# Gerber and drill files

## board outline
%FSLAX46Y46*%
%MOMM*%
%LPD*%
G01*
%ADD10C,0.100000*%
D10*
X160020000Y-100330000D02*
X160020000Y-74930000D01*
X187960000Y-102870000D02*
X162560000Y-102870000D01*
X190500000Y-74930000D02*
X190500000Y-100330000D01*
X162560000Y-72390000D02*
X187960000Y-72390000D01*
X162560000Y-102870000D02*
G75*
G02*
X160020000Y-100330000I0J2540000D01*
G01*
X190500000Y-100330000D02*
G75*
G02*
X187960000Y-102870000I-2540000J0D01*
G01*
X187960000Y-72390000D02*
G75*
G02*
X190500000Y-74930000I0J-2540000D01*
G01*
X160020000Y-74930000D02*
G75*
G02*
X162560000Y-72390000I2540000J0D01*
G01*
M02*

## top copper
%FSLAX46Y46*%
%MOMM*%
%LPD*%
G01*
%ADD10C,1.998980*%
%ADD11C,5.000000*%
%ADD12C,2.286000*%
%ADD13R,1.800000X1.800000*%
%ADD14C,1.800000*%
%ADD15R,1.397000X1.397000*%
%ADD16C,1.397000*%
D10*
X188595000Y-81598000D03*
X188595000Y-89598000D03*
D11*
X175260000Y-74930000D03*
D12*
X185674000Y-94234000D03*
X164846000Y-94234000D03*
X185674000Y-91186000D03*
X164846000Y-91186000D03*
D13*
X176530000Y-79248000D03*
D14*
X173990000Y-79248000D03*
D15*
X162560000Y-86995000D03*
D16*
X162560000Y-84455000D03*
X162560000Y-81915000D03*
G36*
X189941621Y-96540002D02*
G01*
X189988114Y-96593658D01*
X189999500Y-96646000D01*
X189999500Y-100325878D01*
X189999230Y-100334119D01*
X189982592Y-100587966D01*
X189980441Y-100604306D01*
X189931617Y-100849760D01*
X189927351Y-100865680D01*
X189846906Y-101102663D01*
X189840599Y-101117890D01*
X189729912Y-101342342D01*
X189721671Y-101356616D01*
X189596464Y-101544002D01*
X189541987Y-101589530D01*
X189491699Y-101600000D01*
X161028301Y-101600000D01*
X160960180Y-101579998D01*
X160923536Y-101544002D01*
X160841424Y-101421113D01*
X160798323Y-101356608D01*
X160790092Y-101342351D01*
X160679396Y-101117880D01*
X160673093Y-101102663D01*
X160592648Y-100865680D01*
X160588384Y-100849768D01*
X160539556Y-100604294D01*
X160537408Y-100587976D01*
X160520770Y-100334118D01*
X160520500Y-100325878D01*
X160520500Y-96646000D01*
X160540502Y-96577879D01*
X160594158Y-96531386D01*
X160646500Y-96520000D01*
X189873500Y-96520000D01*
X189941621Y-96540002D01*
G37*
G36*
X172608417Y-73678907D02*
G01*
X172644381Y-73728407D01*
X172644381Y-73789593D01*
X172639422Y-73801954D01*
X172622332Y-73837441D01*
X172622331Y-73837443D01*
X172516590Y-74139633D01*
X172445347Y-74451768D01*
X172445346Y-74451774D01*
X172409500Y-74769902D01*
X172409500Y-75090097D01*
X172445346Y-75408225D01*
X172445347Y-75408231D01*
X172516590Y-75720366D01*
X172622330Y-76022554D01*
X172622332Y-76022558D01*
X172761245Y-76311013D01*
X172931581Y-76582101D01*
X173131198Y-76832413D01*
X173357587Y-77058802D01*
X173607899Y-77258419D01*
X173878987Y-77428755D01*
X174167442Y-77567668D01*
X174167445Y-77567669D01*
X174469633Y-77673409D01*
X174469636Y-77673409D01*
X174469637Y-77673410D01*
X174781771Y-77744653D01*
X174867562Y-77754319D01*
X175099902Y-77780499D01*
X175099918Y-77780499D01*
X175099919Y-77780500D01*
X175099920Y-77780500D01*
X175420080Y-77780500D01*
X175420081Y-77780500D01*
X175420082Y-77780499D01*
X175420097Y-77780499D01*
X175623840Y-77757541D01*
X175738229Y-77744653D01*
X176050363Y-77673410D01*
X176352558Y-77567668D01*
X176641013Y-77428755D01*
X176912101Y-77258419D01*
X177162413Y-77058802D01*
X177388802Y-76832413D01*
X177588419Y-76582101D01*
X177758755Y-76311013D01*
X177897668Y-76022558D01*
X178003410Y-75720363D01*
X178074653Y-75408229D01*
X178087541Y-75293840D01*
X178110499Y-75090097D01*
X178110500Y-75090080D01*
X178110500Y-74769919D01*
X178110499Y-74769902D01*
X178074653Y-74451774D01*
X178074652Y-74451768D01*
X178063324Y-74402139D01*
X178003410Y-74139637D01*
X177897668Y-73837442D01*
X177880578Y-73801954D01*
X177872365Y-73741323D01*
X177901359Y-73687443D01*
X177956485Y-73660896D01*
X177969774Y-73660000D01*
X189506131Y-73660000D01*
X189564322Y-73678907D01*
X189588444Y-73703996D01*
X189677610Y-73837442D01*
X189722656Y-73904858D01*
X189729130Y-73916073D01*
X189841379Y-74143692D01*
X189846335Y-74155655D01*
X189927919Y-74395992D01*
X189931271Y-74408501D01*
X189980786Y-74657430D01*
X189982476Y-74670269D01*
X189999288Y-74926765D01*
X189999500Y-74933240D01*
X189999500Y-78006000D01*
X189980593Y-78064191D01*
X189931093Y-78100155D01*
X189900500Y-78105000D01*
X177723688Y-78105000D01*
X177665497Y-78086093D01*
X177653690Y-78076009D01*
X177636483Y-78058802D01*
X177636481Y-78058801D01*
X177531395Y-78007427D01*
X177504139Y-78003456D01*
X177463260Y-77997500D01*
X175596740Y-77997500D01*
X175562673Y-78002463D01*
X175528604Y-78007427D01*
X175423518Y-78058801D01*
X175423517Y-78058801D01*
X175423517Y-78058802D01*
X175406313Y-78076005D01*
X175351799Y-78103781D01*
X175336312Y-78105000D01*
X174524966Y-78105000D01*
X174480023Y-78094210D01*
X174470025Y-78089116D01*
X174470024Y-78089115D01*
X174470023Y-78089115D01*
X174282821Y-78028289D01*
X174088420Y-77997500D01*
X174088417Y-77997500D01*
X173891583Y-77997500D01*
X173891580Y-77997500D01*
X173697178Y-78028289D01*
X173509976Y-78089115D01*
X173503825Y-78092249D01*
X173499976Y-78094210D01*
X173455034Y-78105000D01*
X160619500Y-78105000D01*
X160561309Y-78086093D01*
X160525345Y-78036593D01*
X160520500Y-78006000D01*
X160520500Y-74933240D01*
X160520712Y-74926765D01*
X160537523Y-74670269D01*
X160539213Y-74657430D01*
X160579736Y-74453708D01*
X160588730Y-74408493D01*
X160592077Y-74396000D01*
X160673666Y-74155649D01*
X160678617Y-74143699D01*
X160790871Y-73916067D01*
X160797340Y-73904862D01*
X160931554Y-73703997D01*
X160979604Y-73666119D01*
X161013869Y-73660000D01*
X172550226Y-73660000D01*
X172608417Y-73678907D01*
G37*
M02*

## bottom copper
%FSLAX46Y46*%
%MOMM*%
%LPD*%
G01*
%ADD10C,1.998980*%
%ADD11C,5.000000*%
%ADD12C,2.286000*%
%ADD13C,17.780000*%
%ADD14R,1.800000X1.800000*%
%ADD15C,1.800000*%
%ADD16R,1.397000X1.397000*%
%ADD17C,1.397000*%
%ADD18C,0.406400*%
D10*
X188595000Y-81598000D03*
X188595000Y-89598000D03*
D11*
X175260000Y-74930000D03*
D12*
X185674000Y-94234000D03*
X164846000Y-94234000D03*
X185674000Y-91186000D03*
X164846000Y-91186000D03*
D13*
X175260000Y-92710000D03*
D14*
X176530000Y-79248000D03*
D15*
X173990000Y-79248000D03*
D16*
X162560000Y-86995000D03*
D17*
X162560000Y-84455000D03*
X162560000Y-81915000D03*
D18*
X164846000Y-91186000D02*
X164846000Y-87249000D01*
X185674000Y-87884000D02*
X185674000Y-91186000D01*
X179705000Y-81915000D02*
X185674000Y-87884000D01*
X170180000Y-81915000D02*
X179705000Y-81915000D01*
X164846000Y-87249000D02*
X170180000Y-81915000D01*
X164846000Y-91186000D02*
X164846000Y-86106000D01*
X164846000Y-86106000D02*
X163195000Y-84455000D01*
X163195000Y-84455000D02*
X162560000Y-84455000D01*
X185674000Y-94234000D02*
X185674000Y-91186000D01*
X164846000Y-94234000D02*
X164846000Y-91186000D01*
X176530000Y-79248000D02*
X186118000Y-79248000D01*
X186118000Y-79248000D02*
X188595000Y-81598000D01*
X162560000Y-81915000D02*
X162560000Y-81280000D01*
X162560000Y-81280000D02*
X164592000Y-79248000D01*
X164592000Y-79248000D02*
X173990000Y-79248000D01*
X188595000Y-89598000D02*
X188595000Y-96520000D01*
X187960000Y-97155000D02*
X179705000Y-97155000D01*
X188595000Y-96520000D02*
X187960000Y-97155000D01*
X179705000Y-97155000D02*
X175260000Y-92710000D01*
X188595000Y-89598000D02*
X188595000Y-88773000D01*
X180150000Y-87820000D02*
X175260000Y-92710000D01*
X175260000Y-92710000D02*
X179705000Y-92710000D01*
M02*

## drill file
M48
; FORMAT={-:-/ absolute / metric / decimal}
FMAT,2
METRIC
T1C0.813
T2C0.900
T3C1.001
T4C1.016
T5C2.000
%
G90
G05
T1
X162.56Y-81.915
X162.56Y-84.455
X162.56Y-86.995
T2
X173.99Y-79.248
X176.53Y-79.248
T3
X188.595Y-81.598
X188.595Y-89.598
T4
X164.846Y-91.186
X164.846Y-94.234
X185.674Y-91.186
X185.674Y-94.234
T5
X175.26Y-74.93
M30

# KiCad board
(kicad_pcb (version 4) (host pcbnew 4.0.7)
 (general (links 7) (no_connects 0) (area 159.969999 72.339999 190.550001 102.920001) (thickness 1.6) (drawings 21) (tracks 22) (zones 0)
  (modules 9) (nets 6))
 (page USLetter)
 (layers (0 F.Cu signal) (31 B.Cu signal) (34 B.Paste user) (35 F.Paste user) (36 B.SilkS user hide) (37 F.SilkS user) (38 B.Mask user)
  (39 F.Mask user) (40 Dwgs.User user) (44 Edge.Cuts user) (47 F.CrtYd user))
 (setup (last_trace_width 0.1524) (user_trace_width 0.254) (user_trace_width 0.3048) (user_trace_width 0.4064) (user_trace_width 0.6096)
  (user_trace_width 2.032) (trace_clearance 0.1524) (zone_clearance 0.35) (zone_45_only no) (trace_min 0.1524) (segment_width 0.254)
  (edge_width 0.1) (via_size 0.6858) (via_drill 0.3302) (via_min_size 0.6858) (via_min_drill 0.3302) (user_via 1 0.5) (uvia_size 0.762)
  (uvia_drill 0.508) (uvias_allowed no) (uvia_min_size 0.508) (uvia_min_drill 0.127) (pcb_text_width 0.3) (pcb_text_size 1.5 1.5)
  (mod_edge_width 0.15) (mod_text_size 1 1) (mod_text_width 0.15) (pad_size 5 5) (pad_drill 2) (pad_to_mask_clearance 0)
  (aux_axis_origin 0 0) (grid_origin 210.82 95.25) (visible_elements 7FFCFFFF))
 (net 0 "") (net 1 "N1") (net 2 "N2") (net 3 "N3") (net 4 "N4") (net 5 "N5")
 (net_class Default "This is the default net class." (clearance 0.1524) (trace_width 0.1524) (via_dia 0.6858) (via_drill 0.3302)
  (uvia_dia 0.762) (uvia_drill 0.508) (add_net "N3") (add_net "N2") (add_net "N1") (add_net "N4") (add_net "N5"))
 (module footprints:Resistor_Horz (layer F.Cu) (at 188.595 85.598 270)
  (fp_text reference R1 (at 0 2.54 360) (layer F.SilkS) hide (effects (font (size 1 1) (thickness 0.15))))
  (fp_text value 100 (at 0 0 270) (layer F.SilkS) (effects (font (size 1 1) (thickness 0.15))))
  (pad 1 thru_hole circle (at -4 0 270) (size 1.99898 1.99898) (drill 1.00076) (layers *.Cu *.SilkS *.Mask) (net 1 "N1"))
  (pad 2 thru_hole circle (at 4 0 270) (size 1.99898 1.99898) (drill 1.00076) (layers *.Cu *.SilkS *.Mask) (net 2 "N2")))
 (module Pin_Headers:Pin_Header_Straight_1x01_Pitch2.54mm (layer F.Cu) (at 175.26 74.93)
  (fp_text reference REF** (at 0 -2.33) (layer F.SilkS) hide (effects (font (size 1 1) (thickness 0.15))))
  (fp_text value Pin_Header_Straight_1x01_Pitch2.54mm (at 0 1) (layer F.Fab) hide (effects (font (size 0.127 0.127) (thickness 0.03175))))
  (pad 1 thru_hole circle (at 0 0) (size 5 5) (drill 2) (layers *.Cu B.Mask)))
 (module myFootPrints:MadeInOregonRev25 (layer F.Cu) (at 167.64 76.454)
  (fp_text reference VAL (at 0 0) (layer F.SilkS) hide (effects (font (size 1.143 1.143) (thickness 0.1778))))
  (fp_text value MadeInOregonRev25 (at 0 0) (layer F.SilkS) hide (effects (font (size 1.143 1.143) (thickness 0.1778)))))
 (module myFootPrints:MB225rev (layer F.Cu) (at 184.15 76.2)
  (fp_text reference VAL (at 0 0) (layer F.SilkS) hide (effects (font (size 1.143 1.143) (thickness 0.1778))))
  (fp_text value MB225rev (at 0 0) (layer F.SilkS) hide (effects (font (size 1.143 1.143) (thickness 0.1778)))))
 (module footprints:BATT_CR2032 (layer B.Cu) (at 175.26 92.71 180)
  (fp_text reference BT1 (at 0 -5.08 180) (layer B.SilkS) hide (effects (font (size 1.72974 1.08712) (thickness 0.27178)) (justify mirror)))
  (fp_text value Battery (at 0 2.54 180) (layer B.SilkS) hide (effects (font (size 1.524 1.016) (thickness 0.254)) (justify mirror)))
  (pad 1 thru_hole circle (at -10.414 -1.524 180) (size 2.286 2.286) (drill 1.016) (layers *.Cu *.Mask B.SilkS) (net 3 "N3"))
  (pad 1 thru_hole circle (at 10.414 -1.524 180) (size 2.286 2.286) (drill 1.016) (layers *.Cu *.Mask B.SilkS) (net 3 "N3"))
  (pad 1 thru_hole circle (at -10.414 1.524 180) (size 2.286 2.286) (drill 1.016) (layers *.Cu *.Mask B.SilkS) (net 3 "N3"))
  (pad 1 thru_hole circle (at 10.414 1.524 180) (size 2.286 2.286) (drill 1.016) (layers *.Cu *.Mask B.SilkS) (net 3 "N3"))
  (pad 2 smd circle (at 0 0 180) (size 17.78 17.78) (layers B.Cu B.Paste B.Mask) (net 2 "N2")))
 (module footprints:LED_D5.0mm (layer F.Cu) (at 176.53 79.248 180)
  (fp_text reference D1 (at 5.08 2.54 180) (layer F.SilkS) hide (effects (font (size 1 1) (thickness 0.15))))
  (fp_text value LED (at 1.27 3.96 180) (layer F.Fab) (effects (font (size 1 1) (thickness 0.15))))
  (pad 1 thru_hole rect (at 0 0 180) (size 1.8 1.8) (drill 0.9) (layers *.Cu *.Mask) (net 1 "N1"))
  (pad 2 thru_hole circle (at 2.54 0 180) (size 1.8 1.8) (drill 0.9) (layers *.Cu *.Mask) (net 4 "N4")))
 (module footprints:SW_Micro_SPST (layer F.Cu) (at 162.56 84.455 90)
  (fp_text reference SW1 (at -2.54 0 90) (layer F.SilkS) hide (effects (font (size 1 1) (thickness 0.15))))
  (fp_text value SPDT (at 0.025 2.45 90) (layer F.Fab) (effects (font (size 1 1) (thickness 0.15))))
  (pad 1 thru_hole rect (at -2.54 0 90) (size 1.397 1.397) (drill 0.8128) (layers *.Cu *.Mask F.SilkS) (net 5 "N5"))
  (pad 2 thru_hole circle (at 0 0 90) (size 1.397 1.397) (drill 0.8128) (layers *.Cu *.Mask F.SilkS) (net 3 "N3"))
  (pad 3 thru_hole circle (at 2.54 0 90) (size 1.397 1.397) (drill 0.8128) (layers *.Cu *.Mask F.SilkS) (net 4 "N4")))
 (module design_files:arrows (layer F.Cu) (at 178.308 76.2)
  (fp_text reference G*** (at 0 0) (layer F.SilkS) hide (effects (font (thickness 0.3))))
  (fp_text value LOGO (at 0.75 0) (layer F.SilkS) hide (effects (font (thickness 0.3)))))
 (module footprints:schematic (layer F.Cu) (at 175.26 87.503)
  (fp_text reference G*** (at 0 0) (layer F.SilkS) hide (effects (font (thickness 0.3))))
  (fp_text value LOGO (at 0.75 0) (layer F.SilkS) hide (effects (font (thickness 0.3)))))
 (gr_line (start 160.02 100.33) (end 160.02 74.93) (angle 90) (layer Edge.Cuts) (width 0.1))
 (gr_line (start 187.96 102.87) (end 162.56 102.87) (angle 90) (layer Edge.Cuts) (width 0.1))
 (gr_line (start 190.5 74.93) (end 190.5 100.33) (angle 90) (layer Edge.Cuts) (width 0.1))
 (gr_line (start 162.56 72.39) (end 187.96 72.39) (angle 90) (layer Edge.Cuts) (width 0.1))
 (gr_arc (start 162.56 100.33) (end 162.56 102.87) (angle 90) (layer Edge.Cuts) (width 0.1))
 (gr_arc (start 187.96 100.33) (end 190.5 100.33) (angle 90) (layer Edge.Cuts) (width 0.1))
 (gr_arc (start 187.96 74.93) (end 187.96 72.39) (angle 90) (layer Edge.Cuts) (width 0.1))
 (gr_arc (start 162.56 74.93) (end 160.02 74.93) (angle 90) (layer Edge.Cuts) (width 0.1))
 (segment (start 164.846 91.186) (end 164.846 87.249) (width 0.4064) (layer B.Cu) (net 3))
 (segment (start 185.674 87.884) (end 185.674 91.186) (width 0.4064) (layer B.Cu) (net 3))
 (segment (start 179.705 81.915) (end 185.674 87.884) (width 0.4064) (layer B.Cu) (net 3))
 (segment (start 170.18 81.915) (end 179.705 81.915) (width 0.4064) (layer B.Cu) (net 3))
 (segment (start 164.846 87.249) (end 170.18 81.915) (width 0.4064) (layer B.Cu) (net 3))
 (segment (start 164.846 91.186) (end 164.846 86.106) (width 0.4064) (layer B.Cu) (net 3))
 (segment (start 164.846 86.106) (end 163.195 84.455) (width 0.4064) (layer B.Cu) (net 3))
 (segment (start 163.195 84.455) (end 162.56 84.455) (width 0.4064) (layer B.Cu) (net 3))
 (segment (start 185.674 94.234) (end 185.674 91.186) (width 0.4064) (layer B.Cu) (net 3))
 (segment (start 164.846 94.234) (end 164.846 91.186) (width 0.4064) (layer B.Cu) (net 3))
 (segment (start 176.53 79.248) (end 186.118 79.248) (width 0.4064) (layer B.Cu) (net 1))
 (segment (start 186.118 79.248) (end 188.595 81.598) (width 0.4064) (layer B.Cu) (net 1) (status 20))
 (segment (start 162.56 81.915) (end 162.56 81.28) (width 0.4064) (layer B.Cu) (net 4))
 (segment (start 162.56 81.28) (end 164.592 79.248) (width 0.4064) (layer B.Cu) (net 4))
 (segment (start 164.592 79.248) (end 173.99 79.248) (width 0.4064) (layer B.Cu) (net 4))
 (segment (start 188.595 89.598) (end 188.595 96.52) (width 0.4064) (layer B.Cu) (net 2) (status 10))
 (segment (start 187.96 97.155) (end 179.705 97.155) (width 0.4064) (layer B.Cu) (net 2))
 (segment (start 188.595 96.52) (end 187.96 97.155) (width 0.4064) (layer B.Cu) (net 2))
 (segment (start 179.705 97.155) (end 175.26 92.71) (width 0.4064) (layer B.Cu) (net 2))
 (segment (start 188.595 89.598) (end 188.595 88.773) (width 0.4064) (layer B.Cu) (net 2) (status 30))
 (segment (start 180.15 87.82) (end 175.26 92.71) (width 0.4064) (layer B.Cu) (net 2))
 (segment (start 175.26 92.71) (end 179.705 92.71) (width 0.4064) (layer B.Cu) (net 2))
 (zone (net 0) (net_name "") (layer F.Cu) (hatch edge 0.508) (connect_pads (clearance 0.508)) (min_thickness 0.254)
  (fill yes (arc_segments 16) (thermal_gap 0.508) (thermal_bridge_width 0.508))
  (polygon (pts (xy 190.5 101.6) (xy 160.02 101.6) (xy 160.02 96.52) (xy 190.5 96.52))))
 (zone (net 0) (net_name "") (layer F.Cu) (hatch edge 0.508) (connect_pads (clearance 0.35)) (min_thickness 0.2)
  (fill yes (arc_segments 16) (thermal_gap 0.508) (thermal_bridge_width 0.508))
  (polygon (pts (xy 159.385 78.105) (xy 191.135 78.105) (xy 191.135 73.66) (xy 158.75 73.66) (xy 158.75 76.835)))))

